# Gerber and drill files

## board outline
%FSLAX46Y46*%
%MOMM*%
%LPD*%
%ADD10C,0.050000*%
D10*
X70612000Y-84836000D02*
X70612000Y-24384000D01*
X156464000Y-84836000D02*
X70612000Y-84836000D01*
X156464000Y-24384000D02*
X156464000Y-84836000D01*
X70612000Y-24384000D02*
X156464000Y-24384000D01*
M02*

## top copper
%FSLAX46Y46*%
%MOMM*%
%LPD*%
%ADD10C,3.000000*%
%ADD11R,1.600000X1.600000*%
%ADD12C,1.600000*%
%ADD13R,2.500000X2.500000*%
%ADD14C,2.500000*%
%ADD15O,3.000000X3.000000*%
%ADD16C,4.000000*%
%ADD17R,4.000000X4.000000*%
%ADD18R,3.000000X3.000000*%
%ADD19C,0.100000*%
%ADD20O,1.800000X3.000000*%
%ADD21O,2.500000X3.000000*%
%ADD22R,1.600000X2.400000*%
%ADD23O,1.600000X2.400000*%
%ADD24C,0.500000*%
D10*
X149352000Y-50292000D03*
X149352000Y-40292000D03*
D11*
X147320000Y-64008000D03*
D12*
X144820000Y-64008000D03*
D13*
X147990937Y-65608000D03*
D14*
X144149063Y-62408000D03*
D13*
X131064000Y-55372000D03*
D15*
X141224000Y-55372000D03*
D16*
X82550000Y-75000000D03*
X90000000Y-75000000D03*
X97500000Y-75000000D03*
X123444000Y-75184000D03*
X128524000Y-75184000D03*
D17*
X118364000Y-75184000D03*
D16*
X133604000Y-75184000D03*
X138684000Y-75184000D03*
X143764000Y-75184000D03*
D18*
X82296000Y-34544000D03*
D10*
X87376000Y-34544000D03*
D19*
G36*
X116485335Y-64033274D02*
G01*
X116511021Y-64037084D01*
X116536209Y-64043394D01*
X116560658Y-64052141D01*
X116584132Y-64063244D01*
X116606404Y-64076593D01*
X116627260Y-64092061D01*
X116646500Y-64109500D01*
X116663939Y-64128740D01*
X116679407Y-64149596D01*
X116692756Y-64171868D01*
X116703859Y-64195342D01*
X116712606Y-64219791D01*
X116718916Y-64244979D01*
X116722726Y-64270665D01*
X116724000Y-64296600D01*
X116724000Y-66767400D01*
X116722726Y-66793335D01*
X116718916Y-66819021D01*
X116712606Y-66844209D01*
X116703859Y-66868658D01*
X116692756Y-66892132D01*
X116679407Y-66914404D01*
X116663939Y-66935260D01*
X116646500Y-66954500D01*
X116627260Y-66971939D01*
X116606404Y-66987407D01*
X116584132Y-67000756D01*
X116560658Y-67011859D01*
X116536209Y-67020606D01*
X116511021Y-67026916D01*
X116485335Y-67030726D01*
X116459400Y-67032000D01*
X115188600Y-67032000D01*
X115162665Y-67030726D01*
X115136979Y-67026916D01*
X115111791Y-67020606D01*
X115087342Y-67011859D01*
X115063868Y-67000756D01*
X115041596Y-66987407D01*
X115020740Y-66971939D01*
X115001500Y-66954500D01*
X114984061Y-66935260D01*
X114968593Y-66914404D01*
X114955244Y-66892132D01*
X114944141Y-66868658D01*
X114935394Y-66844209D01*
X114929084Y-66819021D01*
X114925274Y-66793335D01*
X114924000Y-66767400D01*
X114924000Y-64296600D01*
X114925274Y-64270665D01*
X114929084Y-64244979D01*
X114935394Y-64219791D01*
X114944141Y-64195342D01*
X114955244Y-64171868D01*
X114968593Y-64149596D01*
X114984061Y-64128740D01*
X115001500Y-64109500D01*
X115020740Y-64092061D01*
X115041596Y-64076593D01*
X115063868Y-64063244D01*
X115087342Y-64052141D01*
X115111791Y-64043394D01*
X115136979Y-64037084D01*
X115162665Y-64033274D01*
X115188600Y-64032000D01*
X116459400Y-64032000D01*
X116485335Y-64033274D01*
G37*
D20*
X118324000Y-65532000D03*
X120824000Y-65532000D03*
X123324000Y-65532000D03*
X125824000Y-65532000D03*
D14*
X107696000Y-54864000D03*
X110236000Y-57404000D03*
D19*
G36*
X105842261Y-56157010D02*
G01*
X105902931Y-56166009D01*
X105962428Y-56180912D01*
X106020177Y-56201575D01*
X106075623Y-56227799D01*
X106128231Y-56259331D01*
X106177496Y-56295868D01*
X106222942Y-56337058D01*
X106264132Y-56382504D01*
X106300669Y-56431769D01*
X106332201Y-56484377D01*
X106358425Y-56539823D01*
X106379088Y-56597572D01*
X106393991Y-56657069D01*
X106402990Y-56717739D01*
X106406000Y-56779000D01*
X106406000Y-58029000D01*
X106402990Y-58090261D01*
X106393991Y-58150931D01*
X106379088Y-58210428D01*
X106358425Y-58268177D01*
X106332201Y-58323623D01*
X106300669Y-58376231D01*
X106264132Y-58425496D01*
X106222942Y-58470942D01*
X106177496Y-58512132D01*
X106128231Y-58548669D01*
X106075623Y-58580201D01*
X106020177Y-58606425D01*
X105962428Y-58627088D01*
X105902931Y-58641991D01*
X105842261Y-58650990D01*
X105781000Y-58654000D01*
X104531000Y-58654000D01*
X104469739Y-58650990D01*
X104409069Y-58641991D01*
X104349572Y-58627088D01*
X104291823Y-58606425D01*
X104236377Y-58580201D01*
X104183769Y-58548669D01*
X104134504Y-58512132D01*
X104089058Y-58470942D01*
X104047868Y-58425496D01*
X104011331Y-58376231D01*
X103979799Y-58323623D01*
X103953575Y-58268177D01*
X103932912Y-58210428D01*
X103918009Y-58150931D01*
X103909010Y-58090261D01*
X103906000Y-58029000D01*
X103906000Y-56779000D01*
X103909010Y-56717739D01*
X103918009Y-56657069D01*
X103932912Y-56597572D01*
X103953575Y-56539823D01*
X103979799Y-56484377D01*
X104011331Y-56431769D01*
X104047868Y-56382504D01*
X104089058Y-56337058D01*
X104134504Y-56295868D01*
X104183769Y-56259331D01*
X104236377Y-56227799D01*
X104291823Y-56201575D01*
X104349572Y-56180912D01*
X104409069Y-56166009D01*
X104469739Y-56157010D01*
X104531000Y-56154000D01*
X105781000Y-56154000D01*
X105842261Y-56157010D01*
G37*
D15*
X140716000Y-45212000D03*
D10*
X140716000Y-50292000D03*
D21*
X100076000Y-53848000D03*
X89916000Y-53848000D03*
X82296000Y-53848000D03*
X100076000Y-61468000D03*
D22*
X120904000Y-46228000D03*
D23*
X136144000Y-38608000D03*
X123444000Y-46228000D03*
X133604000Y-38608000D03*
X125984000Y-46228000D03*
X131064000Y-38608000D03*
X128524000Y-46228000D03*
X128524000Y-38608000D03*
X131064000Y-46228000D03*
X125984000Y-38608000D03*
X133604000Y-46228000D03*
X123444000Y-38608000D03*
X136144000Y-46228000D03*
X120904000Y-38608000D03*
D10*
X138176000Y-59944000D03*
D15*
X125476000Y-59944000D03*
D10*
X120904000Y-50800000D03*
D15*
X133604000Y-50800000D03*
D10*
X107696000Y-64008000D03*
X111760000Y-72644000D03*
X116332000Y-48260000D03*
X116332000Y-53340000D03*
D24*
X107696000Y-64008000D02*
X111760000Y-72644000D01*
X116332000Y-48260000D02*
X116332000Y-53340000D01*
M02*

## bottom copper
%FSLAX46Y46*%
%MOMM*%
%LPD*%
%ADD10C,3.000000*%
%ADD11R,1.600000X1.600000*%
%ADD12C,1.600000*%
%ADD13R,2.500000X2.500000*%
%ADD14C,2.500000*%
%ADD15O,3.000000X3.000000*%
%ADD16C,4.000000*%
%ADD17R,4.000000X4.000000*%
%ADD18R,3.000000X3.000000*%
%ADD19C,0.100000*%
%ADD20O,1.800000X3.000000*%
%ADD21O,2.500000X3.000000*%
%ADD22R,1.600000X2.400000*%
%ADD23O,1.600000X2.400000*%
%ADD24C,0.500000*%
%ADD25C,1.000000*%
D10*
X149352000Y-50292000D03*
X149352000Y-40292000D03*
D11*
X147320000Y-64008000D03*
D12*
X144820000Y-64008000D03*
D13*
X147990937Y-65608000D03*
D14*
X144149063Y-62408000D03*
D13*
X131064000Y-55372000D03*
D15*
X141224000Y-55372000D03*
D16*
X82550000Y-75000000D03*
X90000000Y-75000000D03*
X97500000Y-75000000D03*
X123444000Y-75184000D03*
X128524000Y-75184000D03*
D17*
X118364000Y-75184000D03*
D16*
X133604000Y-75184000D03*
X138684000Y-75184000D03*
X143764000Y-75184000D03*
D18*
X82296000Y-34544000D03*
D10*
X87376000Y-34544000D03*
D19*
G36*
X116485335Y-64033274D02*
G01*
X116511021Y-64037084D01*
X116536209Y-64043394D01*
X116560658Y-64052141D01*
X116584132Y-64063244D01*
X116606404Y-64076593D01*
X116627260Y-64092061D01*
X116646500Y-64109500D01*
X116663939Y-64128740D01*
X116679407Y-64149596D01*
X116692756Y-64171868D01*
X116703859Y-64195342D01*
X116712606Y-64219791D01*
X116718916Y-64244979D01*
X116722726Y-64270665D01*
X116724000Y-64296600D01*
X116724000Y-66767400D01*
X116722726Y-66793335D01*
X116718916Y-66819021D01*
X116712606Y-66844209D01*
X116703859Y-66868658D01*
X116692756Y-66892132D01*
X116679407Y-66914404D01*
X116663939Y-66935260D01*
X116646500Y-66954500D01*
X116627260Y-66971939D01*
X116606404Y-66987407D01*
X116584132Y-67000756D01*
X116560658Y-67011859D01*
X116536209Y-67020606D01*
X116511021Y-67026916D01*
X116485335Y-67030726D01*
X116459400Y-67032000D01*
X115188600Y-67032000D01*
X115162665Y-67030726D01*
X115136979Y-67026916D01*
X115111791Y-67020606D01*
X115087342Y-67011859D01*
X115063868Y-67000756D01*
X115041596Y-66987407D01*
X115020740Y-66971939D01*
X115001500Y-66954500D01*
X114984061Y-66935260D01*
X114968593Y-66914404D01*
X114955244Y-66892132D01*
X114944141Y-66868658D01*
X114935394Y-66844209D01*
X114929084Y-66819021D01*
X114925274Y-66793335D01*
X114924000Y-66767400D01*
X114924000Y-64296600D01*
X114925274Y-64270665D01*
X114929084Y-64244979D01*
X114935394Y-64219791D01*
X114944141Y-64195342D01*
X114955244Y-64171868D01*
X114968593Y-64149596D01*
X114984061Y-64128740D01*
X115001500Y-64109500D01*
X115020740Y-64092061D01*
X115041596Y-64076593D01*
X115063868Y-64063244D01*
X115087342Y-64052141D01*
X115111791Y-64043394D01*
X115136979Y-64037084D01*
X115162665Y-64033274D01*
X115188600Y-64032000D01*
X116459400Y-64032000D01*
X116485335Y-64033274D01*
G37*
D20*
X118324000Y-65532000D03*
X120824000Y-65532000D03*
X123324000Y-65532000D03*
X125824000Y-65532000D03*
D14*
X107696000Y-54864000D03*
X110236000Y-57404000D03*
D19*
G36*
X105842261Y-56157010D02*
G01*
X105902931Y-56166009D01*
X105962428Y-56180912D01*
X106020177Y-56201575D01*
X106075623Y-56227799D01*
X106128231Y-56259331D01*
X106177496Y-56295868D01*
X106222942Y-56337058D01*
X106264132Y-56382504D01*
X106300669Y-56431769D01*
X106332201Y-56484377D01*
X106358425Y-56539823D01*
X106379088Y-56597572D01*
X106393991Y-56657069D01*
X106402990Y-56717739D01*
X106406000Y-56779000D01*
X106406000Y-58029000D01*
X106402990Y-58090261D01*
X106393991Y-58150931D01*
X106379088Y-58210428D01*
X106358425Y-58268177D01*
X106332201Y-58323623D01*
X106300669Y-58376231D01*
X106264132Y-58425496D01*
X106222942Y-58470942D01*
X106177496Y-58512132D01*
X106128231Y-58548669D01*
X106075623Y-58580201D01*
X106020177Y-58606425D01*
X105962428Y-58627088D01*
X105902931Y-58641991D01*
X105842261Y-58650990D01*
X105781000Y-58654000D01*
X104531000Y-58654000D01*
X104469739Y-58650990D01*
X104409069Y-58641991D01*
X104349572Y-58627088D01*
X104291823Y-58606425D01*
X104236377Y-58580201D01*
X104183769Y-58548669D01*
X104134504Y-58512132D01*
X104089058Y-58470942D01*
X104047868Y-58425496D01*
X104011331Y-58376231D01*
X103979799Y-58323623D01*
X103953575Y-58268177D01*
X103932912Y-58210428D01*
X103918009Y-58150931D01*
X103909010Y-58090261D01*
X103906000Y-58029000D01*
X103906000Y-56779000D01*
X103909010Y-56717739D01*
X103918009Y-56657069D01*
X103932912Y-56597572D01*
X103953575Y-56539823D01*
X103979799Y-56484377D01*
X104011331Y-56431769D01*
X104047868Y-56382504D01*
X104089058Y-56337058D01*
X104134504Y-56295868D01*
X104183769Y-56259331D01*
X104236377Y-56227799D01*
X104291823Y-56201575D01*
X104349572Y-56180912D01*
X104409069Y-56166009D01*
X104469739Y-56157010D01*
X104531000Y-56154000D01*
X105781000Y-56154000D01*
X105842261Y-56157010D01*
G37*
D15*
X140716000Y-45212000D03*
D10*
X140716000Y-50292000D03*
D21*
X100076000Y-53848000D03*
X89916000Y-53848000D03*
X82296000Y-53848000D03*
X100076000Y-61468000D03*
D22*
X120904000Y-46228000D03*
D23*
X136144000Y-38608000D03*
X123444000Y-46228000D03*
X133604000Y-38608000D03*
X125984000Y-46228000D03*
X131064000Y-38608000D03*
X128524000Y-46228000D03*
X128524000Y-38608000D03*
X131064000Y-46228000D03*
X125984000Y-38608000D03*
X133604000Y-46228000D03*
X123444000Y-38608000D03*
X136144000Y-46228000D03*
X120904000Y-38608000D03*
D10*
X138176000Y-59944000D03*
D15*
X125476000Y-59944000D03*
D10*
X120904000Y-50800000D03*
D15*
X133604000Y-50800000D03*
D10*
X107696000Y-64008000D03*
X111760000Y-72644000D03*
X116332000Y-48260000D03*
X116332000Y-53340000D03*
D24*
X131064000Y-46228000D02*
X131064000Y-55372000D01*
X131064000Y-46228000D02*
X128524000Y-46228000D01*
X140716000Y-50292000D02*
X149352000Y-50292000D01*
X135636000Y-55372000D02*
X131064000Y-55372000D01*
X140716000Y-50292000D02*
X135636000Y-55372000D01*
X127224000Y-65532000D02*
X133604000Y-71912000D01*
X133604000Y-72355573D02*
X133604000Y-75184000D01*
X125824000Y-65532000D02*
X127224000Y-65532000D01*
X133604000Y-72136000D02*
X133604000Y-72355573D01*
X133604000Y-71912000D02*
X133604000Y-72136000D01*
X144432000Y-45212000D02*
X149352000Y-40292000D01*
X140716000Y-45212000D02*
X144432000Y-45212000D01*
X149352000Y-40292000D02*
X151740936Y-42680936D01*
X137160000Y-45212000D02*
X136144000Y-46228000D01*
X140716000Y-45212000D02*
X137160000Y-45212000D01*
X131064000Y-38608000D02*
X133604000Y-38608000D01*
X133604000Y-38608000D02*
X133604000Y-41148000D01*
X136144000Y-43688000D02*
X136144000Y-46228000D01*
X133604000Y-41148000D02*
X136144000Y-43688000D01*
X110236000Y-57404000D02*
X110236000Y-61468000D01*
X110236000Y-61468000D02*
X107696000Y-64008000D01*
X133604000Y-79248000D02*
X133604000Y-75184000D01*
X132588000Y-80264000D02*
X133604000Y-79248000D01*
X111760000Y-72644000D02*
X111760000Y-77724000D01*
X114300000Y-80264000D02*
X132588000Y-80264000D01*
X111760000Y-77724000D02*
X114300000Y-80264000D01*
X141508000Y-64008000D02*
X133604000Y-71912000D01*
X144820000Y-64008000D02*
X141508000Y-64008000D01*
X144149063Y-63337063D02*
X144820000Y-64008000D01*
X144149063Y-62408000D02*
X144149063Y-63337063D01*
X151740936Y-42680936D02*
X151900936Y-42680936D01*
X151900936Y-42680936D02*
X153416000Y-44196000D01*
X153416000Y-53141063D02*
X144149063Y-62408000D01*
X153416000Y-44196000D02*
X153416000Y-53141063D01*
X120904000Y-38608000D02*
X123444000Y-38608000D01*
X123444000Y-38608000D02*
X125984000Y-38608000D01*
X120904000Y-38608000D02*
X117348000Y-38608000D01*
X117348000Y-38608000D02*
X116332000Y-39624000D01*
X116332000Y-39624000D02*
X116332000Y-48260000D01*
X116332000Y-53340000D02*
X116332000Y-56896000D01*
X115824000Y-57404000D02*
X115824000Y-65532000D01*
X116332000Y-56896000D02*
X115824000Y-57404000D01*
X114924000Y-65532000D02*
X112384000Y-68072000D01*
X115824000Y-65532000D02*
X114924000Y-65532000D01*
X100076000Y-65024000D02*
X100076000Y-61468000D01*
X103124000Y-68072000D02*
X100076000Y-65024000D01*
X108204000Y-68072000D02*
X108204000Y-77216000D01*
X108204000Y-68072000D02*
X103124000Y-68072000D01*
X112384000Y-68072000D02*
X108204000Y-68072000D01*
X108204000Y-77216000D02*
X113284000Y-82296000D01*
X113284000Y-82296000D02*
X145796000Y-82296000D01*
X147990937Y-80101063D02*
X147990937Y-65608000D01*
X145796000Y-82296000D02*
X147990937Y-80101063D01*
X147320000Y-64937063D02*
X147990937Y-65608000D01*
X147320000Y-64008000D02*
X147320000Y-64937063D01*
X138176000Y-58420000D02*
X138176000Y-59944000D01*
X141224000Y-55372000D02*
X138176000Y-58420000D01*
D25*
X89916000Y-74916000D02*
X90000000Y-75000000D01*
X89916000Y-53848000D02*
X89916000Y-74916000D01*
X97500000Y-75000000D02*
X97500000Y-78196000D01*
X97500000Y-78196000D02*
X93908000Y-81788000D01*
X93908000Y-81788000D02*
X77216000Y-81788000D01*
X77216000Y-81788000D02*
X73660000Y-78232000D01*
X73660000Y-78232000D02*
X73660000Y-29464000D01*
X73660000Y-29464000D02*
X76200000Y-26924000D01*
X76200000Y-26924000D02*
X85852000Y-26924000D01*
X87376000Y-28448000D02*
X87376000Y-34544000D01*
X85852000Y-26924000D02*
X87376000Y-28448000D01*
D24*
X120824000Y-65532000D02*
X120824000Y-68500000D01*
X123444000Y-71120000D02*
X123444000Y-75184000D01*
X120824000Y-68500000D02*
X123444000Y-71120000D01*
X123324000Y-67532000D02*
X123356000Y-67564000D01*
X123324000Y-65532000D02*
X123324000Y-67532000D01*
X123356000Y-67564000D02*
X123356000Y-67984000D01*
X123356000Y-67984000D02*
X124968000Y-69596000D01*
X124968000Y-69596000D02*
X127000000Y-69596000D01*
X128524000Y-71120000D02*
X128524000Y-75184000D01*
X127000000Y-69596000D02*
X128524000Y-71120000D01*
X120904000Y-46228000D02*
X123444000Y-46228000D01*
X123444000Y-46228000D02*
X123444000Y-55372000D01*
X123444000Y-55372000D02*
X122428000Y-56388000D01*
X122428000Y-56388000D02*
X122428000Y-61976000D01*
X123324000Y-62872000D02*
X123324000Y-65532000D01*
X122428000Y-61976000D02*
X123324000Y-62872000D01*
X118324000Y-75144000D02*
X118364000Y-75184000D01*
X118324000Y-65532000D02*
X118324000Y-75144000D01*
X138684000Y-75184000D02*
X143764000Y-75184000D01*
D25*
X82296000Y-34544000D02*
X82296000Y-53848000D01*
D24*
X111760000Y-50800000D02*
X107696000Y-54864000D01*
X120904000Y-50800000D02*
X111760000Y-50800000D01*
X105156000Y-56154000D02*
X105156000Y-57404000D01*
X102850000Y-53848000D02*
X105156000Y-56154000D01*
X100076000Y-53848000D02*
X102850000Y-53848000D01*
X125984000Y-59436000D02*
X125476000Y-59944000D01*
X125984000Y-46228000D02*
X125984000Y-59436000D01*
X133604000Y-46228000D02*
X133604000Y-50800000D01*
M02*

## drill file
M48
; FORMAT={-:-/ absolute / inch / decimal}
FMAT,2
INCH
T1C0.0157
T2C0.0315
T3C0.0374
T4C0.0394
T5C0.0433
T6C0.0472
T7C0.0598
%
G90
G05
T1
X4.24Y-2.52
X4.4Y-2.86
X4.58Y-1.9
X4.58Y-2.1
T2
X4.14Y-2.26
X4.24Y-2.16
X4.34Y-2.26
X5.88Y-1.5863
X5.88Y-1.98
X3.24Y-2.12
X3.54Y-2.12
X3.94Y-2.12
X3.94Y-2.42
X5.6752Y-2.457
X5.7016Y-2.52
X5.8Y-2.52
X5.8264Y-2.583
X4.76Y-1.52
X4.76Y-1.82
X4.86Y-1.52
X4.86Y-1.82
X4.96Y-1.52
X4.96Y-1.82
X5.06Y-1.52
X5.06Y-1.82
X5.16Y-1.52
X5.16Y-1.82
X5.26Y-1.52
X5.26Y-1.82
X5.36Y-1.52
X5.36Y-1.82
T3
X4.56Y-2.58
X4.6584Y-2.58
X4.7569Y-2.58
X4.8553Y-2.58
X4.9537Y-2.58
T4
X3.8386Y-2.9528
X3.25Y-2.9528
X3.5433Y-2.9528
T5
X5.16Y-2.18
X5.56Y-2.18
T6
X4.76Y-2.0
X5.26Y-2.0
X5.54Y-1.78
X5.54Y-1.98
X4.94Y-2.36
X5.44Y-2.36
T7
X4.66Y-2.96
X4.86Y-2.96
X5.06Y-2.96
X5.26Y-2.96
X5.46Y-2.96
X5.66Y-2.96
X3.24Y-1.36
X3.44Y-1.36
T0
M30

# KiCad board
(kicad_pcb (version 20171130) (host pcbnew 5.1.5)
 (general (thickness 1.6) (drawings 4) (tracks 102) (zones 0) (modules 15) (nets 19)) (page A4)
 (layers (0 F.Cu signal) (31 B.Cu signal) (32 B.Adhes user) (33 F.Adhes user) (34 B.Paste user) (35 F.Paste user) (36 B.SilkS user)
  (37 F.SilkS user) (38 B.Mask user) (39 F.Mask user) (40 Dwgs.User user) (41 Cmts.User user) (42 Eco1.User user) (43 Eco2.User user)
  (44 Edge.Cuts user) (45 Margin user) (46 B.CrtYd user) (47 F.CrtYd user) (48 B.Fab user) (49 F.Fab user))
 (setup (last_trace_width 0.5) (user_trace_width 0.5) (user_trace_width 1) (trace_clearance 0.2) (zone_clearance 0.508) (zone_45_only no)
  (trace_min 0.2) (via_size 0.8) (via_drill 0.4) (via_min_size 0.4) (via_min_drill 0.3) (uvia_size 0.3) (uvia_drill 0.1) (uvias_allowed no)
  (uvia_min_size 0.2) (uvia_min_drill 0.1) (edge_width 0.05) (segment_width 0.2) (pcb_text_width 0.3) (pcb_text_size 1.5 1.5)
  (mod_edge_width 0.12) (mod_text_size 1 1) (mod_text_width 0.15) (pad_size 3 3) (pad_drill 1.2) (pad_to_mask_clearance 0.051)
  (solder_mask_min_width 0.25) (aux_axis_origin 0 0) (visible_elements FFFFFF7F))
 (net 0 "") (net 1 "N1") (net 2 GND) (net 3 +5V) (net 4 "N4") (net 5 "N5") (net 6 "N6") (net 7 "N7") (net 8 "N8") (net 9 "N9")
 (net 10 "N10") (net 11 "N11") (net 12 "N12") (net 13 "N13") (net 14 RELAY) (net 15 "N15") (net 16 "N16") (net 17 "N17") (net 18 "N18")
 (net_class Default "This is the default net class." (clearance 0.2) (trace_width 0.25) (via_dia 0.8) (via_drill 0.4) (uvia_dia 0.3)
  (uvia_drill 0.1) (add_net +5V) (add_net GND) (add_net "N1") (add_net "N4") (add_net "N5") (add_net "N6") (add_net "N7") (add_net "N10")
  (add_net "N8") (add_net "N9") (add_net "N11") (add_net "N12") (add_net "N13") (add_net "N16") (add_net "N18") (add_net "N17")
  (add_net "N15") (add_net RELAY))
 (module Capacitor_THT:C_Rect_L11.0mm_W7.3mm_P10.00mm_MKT (layer F.Cu) (at 149.352 50.292 90)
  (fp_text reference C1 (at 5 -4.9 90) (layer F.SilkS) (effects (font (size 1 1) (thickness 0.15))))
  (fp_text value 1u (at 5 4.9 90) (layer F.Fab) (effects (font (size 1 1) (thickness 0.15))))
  (pad 1 thru_hole circle (at 0 0 90) (size 3 3) (drill 0.8) (layers *.Cu *.Mask) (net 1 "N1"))
  (pad 2 thru_hole circle (at 10 0 90) (size 3 3) (drill 0.8) (layers *.Cu *.Mask) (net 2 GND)))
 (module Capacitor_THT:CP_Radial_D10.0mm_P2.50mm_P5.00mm (layer F.Cu) (at 147.32 64.008 180)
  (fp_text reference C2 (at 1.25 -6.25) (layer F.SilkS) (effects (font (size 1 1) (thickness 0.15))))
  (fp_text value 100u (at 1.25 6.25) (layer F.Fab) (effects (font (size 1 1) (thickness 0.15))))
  (pad 1 thru_hole rect (at 0 0 180) (size 1.6 1.6) (drill 0.8) (layers *.Cu *.Mask) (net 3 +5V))
  (pad 2 thru_hole circle (at 2.5 0 180) (size 1.6 1.6) (drill 0.8) (layers *.Cu *.Mask) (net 2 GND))
  (pad 1 thru_hole rect (at -0.670937 -1.6 180) (size 2.5 2.5) (drill 0.8) (layers *.Cu *.Mask) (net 3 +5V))
  (pad 2 thru_hole circle (at 3.170937 1.6 180) (size 2.5 2.5) (drill 0.8) (layers *.Cu *.Mask) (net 2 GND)))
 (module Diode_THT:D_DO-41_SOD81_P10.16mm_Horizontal (layer F.Cu) (at 131.064 55.372)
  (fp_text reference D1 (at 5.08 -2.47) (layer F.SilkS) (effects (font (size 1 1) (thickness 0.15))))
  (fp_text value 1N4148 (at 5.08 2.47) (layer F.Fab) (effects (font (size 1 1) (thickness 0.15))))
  (pad 1 thru_hole rect (at 0 0) (size 2.5 2.5) (drill 1.1) (layers *.Cu *.Mask) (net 1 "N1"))
  (pad 2 thru_hole oval (at 10.16 0) (size 3 3) (drill 1.1) (layers *.Cu *.Mask) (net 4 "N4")))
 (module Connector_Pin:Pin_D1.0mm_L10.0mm (layer F.Cu) (at 82.55 75)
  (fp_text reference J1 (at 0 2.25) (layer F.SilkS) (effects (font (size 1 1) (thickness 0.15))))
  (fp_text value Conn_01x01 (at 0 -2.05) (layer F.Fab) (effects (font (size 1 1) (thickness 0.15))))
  (pad 1 thru_hole circle (at 0 0) (size 4 4) (drill 1) (layers *.Cu *.Mask) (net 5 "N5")))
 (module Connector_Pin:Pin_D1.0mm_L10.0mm (layer F.Cu) (at 90 75)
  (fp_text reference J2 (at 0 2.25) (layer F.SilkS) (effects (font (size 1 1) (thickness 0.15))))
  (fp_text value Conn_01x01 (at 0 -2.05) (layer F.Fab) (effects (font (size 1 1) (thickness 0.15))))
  (pad 1 thru_hole circle (at 0 0) (size 4 4) (drill 1) (layers *.Cu *.Mask) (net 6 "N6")))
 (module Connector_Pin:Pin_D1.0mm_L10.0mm (layer F.Cu) (at 97.5 75)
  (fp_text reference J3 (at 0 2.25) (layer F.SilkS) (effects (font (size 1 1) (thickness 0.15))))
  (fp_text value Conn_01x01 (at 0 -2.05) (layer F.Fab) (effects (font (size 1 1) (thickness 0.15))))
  (pad 1 thru_hole circle (at 0 0) (size 4 4) (drill 1) (layers *.Cu *.Mask) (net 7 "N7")))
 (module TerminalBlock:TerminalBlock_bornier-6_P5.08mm (layer F.Cu) (at 118.364 75.184)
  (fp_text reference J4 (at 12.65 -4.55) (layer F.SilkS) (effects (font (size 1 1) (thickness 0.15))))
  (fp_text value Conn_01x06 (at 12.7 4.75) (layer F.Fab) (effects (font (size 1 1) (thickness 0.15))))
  (pad 2 thru_hole circle (at 5.08 0) (size 4 4) (drill 1.52) (layers *.Cu *.Mask) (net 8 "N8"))
  (pad 3 thru_hole circle (at 10.16 0) (size 4 4) (drill 1.52) (layers *.Cu *.Mask) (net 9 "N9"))
  (pad 1 thru_hole rect (at 0 0) (size 4 4) (drill 1.52) (layers *.Cu *.Mask) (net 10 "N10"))
  (pad 4 thru_hole circle (at 15.24 0) (size 4 4) (drill 1.52) (layers *.Cu *.Mask) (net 2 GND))
  (pad 5 thru_hole circle (at 20.32 0) (size 4 4) (drill 1.52) (layers *.Cu *.Mask) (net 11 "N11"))
  (pad 6 thru_hole circle (at 25.4 0) (size 4 4) (drill 1.52) (layers *.Cu *.Mask) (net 11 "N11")))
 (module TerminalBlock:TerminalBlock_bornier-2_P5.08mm (layer F.Cu) (at 82.296 34.544)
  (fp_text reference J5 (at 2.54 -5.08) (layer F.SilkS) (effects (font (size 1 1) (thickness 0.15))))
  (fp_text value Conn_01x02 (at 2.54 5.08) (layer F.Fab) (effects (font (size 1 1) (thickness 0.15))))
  (pad 1 thru_hole rect (at 0 0) (size 3 3) (drill 1.52) (layers *.Cu *.Mask) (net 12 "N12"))
  (pad 2 thru_hole circle (at 5.08 0) (size 3 3) (drill 1.52) (layers *.Cu *.Mask) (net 7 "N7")))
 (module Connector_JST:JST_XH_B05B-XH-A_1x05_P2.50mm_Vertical (layer F.Cu) (at 115.824 65.532)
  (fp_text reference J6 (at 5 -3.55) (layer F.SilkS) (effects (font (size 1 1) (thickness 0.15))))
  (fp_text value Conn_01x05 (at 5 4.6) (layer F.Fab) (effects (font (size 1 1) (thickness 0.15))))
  (pad 1 thru_hole roundrect (at 0 0) (size 1.8 3) (drill 0.95) (layers *.Cu *.Mask) (roundrect_rratio 0.147) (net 3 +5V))
  (pad 2 thru_hole oval (at 2.5 0) (size 1.8 3) (drill 0.95) (layers *.Cu *.Mask) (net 10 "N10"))
  (pad 3 thru_hole oval (at 5 0) (size 1.8 3) (drill 0.95) (layers *.Cu *.Mask) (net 8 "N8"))
  (pad 4 thru_hole oval (at 7.5 0) (size 1.8 3) (drill 0.95) (layers *.Cu *.Mask) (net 9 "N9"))
  (pad 5 thru_hole oval (at 10 0) (size 1.8 3) (drill 0.95) (layers *.Cu *.Mask) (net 2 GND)))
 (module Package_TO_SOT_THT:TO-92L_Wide (layer F.Cu) (at 105.156 57.404)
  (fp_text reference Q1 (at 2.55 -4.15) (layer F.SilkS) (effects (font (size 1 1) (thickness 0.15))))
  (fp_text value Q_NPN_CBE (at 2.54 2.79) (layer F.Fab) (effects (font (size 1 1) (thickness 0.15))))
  (pad 2 thru_hole circle (at 2.54 -2.54 90) (size 2.5 2.5) (drill 0.8) (layers *.Cu *.Mask) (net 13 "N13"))
  (pad 3 thru_hole circle (at 5.08 0 90) (size 2.5 2.5) (drill 0.8) (layers *.Cu *.Mask) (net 2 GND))
  (pad 1 thru_hole roundrect (at 0 0 90) (size 2.5 2.5) (drill 0.8) (layers *.Cu *.Mask) (roundrect_rratio 0.25) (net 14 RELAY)))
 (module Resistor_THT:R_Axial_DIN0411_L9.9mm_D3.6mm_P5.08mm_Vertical (layer F.Cu) (at 140.716 50.292 90)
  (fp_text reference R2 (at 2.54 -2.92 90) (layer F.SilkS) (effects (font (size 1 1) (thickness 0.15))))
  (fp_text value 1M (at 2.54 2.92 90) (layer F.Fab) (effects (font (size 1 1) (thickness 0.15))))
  (pad 2 thru_hole oval (at 5.08 0 90) (size 3 3) (drill 1.2) (layers *.Cu *.Mask) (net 2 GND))
  (pad 1 thru_hole circle (at 0 0 90) (size 3 3) (drill 1.2) (layers *.Cu *.Mask) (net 1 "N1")))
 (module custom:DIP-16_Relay (layer F.Cu) (at 100.076 53.848 270)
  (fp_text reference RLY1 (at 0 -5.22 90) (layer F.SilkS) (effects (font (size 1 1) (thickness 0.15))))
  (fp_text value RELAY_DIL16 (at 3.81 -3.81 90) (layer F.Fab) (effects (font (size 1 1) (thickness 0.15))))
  (pad 1 thru_hole oval (at 0 0 270) (size 3 2.5) (drill 0.8) (layers *.Cu *.Mask F.SilkS) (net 14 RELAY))
  (pad 5 thru_hole oval (at 0 10.16 270) (size 3 2.5) (drill 0.8) (layers *.Cu *.Mask F.SilkS) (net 6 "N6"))
  (pad 8 thru_hole oval (at 0 17.78 270) (size 3 2.5) (drill 0.8) (layers *.Cu *.Mask F.SilkS) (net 12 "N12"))
  (pad 16 thru_hole oval (at 7.62 0 270) (size 3 2.5) (drill 0.8) (layers *.Cu *.Mask F.SilkS) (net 3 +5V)))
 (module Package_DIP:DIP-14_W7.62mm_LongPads (layer F.Cu) (at 120.904 46.228 90)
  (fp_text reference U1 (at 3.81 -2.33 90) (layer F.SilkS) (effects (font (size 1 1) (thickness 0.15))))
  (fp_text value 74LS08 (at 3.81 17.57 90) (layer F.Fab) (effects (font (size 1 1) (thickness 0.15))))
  (pad 1 thru_hole rect (at 0 0 90) (size 2.4 1.6) (drill 0.8) (layers *.Cu *.Mask) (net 9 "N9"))
  (pad 8 thru_hole oval (at 7.62 15.24 90) (size 2.4 1.6) (drill 0.8) (layers *.Cu *.Mask) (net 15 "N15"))
  (pad 2 thru_hole oval (at 0 2.54 90) (size 2.4 1.6) (drill 0.8) (layers *.Cu *.Mask) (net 9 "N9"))
  (pad 9 thru_hole oval (at 7.62 12.7 90) (size 2.4 1.6) (drill 0.8) (layers *.Cu *.Mask) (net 2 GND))
  (pad 3 thru_hole oval (at 0 5.08 90) (size 2.4 1.6) (drill 0.8) (layers *.Cu *.Mask) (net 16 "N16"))
  (pad 10 thru_hole oval (at 7.62 10.16 90) (size 2.4 1.6) (drill 0.8) (layers *.Cu *.Mask) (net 2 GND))
  (pad 4 thru_hole oval (at 0 7.62 90) (size 2.4 1.6) (drill 0.8) (layers *.Cu *.Mask) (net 1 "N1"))
  (pad 11 thru_hole oval (at 7.62 7.62 90) (size 2.4 1.6) (drill 0.8) (layers *.Cu *.Mask) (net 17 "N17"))
  (pad 5 thru_hole oval (at 0 10.16 90) (size 2.4 1.6) (drill 0.8) (layers *.Cu *.Mask) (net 1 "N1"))
  (pad 12 thru_hole oval (at 7.62 5.08 90) (size 2.4 1.6) (drill 0.8) (layers *.Cu *.Mask) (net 3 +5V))
  (pad 6 thru_hole oval (at 0 12.7 90) (size 2.4 1.6) (drill 0.8) (layers *.Cu *.Mask) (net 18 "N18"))
  (pad 13 thru_hole oval (at 7.62 2.54 90) (size 2.4 1.6) (drill 0.8) (layers *.Cu *.Mask) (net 3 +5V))
  (pad 7 thru_hole oval (at 0 15.24 90) (size 2.4 1.6) (drill 0.8) (layers *.Cu *.Mask) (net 2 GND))
  (pad 14 thru_hole oval (at 7.62 0 90) (size 2.4 1.6) (drill 0.8) (layers *.Cu *.Mask) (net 3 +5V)))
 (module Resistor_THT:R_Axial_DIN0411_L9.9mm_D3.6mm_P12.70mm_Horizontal (layer F.Cu) (at 138.176 59.944 180)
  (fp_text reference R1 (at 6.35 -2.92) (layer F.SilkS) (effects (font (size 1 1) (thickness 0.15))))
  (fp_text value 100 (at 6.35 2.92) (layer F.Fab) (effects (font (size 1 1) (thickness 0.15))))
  (pad 1 thru_hole circle (at 0 0 180) (size 3 3) (drill 1.2) (layers *.Cu *.Mask) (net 4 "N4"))
  (pad 2 thru_hole oval (at 12.7 0 180) (size 3 3) (drill 1.2) (layers *.Cu *.Mask) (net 16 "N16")))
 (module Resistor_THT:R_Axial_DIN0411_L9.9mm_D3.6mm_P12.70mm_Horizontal (layer F.Cu) (at 120.904 50.8)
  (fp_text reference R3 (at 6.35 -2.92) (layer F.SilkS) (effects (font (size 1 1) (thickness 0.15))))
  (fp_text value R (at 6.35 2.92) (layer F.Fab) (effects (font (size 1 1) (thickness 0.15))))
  (pad 1 thru_hole circle (at 0 0) (size 3 3) (drill 1.2) (layers *.Cu *.Mask) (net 13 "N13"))
  (pad 2 thru_hole oval (at 12.7 0) (size 3 3) (drill 1.2) (layers *.Cu *.Mask) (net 18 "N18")))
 (gr_line (start 70.612 84.836) (end 70.612 24.384) (layer Edge.Cuts) (width 0.05))
 (gr_line (start 156.464 84.836) (end 70.612 84.836) (layer Edge.Cuts) (width 0.05))
 (gr_line (start 156.464 24.384) (end 156.464 84.836) (layer Edge.Cuts) (width 0.05))
 (gr_line (start 70.612 24.384) (end 156.464 24.384) (layer Edge.Cuts) (width 0.05))
 (segment (start 131.064 46.228) (end 131.064 55.372) (width 0.5) (layer B.Cu) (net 1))
 (segment (start 131.064 46.228) (end 128.524 46.228) (width 0.5) (layer B.Cu) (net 1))
 (segment (start 140.716 50.292) (end 149.352 50.292) (width 0.5) (layer B.Cu) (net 1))
 (segment (start 135.636 55.372) (end 131.064 55.372) (width 0.5) (layer B.Cu) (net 1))
 (segment (start 140.716 50.292) (end 135.636 55.372) (width 0.5) (layer B.Cu) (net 1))
 (segment (start 127.224 65.532) (end 133.604 71.912) (width 0.5) (layer B.Cu) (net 2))
 (segment (start 133.604 72.355573) (end 133.604 75.184) (width 0.5) (layer B.Cu) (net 2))
 (segment (start 125.824 65.532) (end 127.224 65.532) (width 0.5) (layer B.Cu) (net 2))
 (segment (start 133.604 72.136) (end 133.604 72.355573) (width 0.5) (layer B.Cu) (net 2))
 (segment (start 133.604 71.912) (end 133.604 72.136) (width 0.5) (layer B.Cu) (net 2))
 (segment (start 144.432 45.212) (end 149.352 40.292) (width 0.5) (layer B.Cu) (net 2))
 (segment (start 140.716 45.212) (end 144.432 45.212) (width 0.5) (layer B.Cu) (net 2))
 (segment (start 149.352 40.292) (end 151.740936 42.680936) (width 0.5) (layer B.Cu) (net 2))
 (segment (start 137.16 45.212) (end 136.144 46.228) (width 0.5) (layer B.Cu) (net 2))
 (segment (start 140.716 45.212) (end 137.16 45.212) (width 0.5) (layer B.Cu) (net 2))
 (segment (start 131.064 38.608) (end 133.604 38.608) (width 0.5) (layer B.Cu) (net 2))
 (segment (start 133.604 38.608) (end 133.604 41.148) (width 0.5) (layer B.Cu) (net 2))
 (segment (start 136.144 43.688) (end 136.144 46.228) (width 0.5) (layer B.Cu) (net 2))
 (segment (start 133.604 41.148) (end 136.144 43.688) (width 0.5) (layer B.Cu) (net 2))
 (via (at 107.696 64.008) (size 3) (drill 0.4) (layers F.Cu B.Cu) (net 2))
 (segment (start 110.236 57.404) (end 110.236 61.468) (width 0.5) (layer B.Cu) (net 2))
 (segment (start 110.236 61.468) (end 107.696 64.008) (width 0.5) (layer B.Cu) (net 2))
 (segment (start 107.696 64.008) (end 111.76 72.644) (width 0.5) (layer F.Cu) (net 2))
 (via (at 111.76 72.644) (size 3) (drill 0.4) (layers F.Cu B.Cu) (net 2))
 (segment (start 133.604 79.248) (end 133.604 75.184) (width 0.5) (layer B.Cu) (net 2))
 (segment (start 132.588 80.264) (end 133.604 79.248) (width 0.5) (layer B.Cu) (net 2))
 (segment (start 111.76 72.644) (end 111.76 77.724) (width 0.5) (layer B.Cu) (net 2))
 (segment (start 114.3 80.264) (end 132.588 80.264) (width 0.5) (layer B.Cu) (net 2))
 (segment (start 111.76 77.724) (end 114.3 80.264) (width 0.5) (layer B.Cu) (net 2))
 (segment (start 141.508 64.008) (end 133.604 71.912) (width 0.5) (layer B.Cu) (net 2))
 (segment (start 144.82 64.008) (end 141.508 64.008) (width 0.5) (layer B.Cu) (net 2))
 (segment (start 144.149063 63.337063) (end 144.82 64.008) (width 0.5) (layer B.Cu) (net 2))
 (segment (start 144.149063 62.408) (end 144.149063 63.337063) (width 0.5) (layer B.Cu) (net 2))
 (segment (start 151.740936 42.680936) (end 151.900936 42.680936) (width 0.5) (layer B.Cu) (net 2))
 (segment (start 151.900936 42.680936) (end 153.416 44.196) (width 0.5) (layer B.Cu) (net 2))
 (segment (start 153.416 53.141063) (end 144.149063 62.408) (width 0.5) (layer B.Cu) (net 2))
 (segment (start 153.416 44.196) (end 153.416 53.141063) (width 0.5) (layer B.Cu) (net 2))
 (segment (start 120.904 38.608) (end 123.444 38.608) (width 0.5) (layer B.Cu) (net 3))
 (segment (start 123.444 38.608) (end 125.984 38.608) (width 0.5) (layer B.Cu) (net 3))
 (segment (start 120.904 38.608) (end 117.348 38.608) (width 0.5) (layer B.Cu) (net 3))
 (via (at 116.332 48.26) (size 3) (drill 0.4) (layers F.Cu B.Cu) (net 3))
 (segment (start 117.348 38.608) (end 116.332 39.624) (width 0.5) (layer B.Cu) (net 3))
 (segment (start 116.332 39.624) (end 116.332 48.26) (width 0.5) (layer B.Cu) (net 3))
 (via (at 116.332 53.34) (size 3) (drill 0.4) (layers F.Cu B.Cu) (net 3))
 (segment (start 116.332 48.26) (end 116.332 53.34) (width 0.5) (layer F.Cu) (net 3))
 (segment (start 116.332 53.34) (end 116.332 56.896) (width 0.5) (layer B.Cu) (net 3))
 (segment (start 115.824 57.404) (end 115.824 65.532) (width 0.5) (layer B.Cu) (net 3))
 (segment (start 116.332 56.896) (end 115.824 57.404) (width 0.5) (layer B.Cu) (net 3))
 (segment (start 114.924 65.532) (end 112.384 68.072) (width 0.5) (layer B.Cu) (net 3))
 (segment (start 115.824 65.532) (end 114.924 65.532) (width 0.5) (layer B.Cu) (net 3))
 (segment (start 100.076 65.024) (end 100.076 61.468) (width 0.5) (layer B.Cu) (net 3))
 (segment (start 103.124 68.072) (end 100.076 65.024) (width 0.5) (layer B.Cu) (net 3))
 (segment (start 108.204 68.072) (end 108.204 77.216) (width 0.5) (layer B.Cu) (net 3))
 (segment (start 108.204 68.072) (end 103.124 68.072) (width 0.5) (layer B.Cu) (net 3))
 (segment (start 112.384 68.072) (end 108.204 68.072) (width 0.5) (layer B.Cu) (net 3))
 (segment (start 108.204 77.216) (end 113.284 82.296) (width 0.5) (layer B.Cu) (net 3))
 (segment (start 113.284 82.296) (end 145.796 82.296) (width 0.5) (layer B.Cu) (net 3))
 (segment (start 147.990937 80.101063) (end 147.990937 65.608) (width 0.5) (layer B.Cu) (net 3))
 (segment (start 145.796 82.296) (end 147.990937 80.101063) (width 0.5) (layer B.Cu) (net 3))
 (segment (start 147.32 64.937063) (end 147.990937 65.608) (width 0.5) (layer B.Cu) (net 3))
 (segment (start 147.32 64.008) (end 147.32 64.937063) (width 0.5) (layer B.Cu) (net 3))
 (segment (start 138.176 58.42) (end 138.176 59.944) (width 0.5) (layer B.Cu) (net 4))
 (segment (start 141.224 55.372) (end 138.176 58.42) (width 0.5) (layer B.Cu) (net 4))
 (segment (start 89.916 74.916) (end 90 75) (width 1) (layer B.Cu) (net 6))
 (segment (start 89.916 53.848) (end 89.916 74.916) (width 1) (layer B.Cu) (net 6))
 (segment (start 97.5 75) (end 97.5 78.196) (width 1) (layer B.Cu) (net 7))
 (segment (start 97.5 78.196) (end 93.908 81.788) (width 1) (layer B.Cu) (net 7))
 (segment (start 93.908 81.788) (end 77.216 81.788) (width 1) (layer B.Cu) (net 7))
 (segment (start 77.216 81.788) (end 73.66 78.232) (width 1) (layer B.Cu) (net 7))
 (segment (start 73.66 78.232) (end 73.66 29.464) (width 1) (layer B.Cu) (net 7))
 (segment (start 73.66 29.464) (end 76.2 26.924) (width 1) (layer B.Cu) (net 7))
 (segment (start 76.2 26.924) (end 85.852 26.924) (width 1) (layer B.Cu) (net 7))
 (segment (start 87.376 28.448) (end 87.376 34.544) (width 1) (layer B.Cu) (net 7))
 (segment (start 85.852 26.924) (end 87.376 28.448) (width 1) (layer B.Cu) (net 7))
 (segment (start 120.824 65.532) (end 120.824 68.5) (width 0.5) (layer B.Cu) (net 8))
 (segment (start 123.444 71.12) (end 123.444 75.184) (width 0.5) (layer B.Cu) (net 8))
 (segment (start 120.824 68.5) (end 123.444 71.12) (width 0.5) (layer B.Cu) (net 8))
 (segment (start 123.324 67.532) (end 123.356 67.564) (width 0.5) (layer B.Cu) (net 9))
 (segment (start 123.324 65.532) (end 123.324 67.532) (width 0.5) (layer B.Cu) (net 9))
 (segment (start 123.356 67.564) (end 123.356 67.984) (width 0.5) (layer B.Cu) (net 9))
 (segment (start 123.356 67.984) (end 124.968 69.596) (width 0.5) (layer B.Cu) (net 9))
 (segment (start 124.968 69.596) (end 127 69.596) (width 0.5) (layer B.Cu) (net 9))
 (segment (start 128.524 71.12) (end 128.524 75.184) (width 0.5) (layer B.Cu) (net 9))
 (segment (start 127 69.596) (end 128.524 71.12) (width 0.5) (layer B.Cu) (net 9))
 (segment (start 120.904 46.228) (end 123.444 46.228) (width 0.5) (layer B.Cu) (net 9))
 (segment (start 123.444 46.228) (end 123.444 55.372) (width 0.5) (layer B.Cu) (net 9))
 (segment (start 123.444 55.372) (end 122.428 56.388) (width 0.5) (layer B.Cu) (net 9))
 (segment (start 122.428 56.388) (end 122.428 61.976) (width 0.5) (layer B.Cu) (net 9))
 (segment (start 123.324 62.872) (end 123.324 65.532) (width 0.5) (layer B.Cu) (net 9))
 (segment (start 122.428 61.976) (end 123.324 62.872) (width 0.5) (layer B.Cu) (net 9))
 (segment (start 118.324 75.144) (end 118.364 75.184) (width 0.5) (layer B.Cu) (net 10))
 (segment (start 118.324 65.532) (end 118.324 75.144) (width 0.5) (layer B.Cu) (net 10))
 (segment (start 138.684 75.184) (end 143.764 75.184) (width 0.5) (layer B.Cu) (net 11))
 (segment (start 82.296 34.544) (end 82.296 53.848) (width 1) (layer B.Cu) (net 12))
 (segment (start 111.76 50.8) (end 107.696 54.864) (width 0.5) (layer B.Cu) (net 13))
 (segment (start 120.904 50.8) (end 111.76 50.8) (width 0.5) (layer B.Cu) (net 13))
 (segment (start 105.156 56.154) (end 105.156 57.404) (width 0.5) (layer B.Cu) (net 14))
 (segment (start 102.85 53.848) (end 105.156 56.154) (width 0.5) (layer B.Cu) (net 14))
 (segment (start 100.076 53.848) (end 102.85 53.848) (width 0.5) (layer B.Cu) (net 14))
 (segment (start 125.984 59.436) (end 125.476 59.944) (width 0.5) (layer B.Cu) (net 16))
 (segment (start 125.984 46.228) (end 125.984 59.436) (width 0.5) (layer B.Cu) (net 16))
 (segment (start 133.604 46.228) (end 133.604 50.8) (width 0.5) (layer B.Cu) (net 18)))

